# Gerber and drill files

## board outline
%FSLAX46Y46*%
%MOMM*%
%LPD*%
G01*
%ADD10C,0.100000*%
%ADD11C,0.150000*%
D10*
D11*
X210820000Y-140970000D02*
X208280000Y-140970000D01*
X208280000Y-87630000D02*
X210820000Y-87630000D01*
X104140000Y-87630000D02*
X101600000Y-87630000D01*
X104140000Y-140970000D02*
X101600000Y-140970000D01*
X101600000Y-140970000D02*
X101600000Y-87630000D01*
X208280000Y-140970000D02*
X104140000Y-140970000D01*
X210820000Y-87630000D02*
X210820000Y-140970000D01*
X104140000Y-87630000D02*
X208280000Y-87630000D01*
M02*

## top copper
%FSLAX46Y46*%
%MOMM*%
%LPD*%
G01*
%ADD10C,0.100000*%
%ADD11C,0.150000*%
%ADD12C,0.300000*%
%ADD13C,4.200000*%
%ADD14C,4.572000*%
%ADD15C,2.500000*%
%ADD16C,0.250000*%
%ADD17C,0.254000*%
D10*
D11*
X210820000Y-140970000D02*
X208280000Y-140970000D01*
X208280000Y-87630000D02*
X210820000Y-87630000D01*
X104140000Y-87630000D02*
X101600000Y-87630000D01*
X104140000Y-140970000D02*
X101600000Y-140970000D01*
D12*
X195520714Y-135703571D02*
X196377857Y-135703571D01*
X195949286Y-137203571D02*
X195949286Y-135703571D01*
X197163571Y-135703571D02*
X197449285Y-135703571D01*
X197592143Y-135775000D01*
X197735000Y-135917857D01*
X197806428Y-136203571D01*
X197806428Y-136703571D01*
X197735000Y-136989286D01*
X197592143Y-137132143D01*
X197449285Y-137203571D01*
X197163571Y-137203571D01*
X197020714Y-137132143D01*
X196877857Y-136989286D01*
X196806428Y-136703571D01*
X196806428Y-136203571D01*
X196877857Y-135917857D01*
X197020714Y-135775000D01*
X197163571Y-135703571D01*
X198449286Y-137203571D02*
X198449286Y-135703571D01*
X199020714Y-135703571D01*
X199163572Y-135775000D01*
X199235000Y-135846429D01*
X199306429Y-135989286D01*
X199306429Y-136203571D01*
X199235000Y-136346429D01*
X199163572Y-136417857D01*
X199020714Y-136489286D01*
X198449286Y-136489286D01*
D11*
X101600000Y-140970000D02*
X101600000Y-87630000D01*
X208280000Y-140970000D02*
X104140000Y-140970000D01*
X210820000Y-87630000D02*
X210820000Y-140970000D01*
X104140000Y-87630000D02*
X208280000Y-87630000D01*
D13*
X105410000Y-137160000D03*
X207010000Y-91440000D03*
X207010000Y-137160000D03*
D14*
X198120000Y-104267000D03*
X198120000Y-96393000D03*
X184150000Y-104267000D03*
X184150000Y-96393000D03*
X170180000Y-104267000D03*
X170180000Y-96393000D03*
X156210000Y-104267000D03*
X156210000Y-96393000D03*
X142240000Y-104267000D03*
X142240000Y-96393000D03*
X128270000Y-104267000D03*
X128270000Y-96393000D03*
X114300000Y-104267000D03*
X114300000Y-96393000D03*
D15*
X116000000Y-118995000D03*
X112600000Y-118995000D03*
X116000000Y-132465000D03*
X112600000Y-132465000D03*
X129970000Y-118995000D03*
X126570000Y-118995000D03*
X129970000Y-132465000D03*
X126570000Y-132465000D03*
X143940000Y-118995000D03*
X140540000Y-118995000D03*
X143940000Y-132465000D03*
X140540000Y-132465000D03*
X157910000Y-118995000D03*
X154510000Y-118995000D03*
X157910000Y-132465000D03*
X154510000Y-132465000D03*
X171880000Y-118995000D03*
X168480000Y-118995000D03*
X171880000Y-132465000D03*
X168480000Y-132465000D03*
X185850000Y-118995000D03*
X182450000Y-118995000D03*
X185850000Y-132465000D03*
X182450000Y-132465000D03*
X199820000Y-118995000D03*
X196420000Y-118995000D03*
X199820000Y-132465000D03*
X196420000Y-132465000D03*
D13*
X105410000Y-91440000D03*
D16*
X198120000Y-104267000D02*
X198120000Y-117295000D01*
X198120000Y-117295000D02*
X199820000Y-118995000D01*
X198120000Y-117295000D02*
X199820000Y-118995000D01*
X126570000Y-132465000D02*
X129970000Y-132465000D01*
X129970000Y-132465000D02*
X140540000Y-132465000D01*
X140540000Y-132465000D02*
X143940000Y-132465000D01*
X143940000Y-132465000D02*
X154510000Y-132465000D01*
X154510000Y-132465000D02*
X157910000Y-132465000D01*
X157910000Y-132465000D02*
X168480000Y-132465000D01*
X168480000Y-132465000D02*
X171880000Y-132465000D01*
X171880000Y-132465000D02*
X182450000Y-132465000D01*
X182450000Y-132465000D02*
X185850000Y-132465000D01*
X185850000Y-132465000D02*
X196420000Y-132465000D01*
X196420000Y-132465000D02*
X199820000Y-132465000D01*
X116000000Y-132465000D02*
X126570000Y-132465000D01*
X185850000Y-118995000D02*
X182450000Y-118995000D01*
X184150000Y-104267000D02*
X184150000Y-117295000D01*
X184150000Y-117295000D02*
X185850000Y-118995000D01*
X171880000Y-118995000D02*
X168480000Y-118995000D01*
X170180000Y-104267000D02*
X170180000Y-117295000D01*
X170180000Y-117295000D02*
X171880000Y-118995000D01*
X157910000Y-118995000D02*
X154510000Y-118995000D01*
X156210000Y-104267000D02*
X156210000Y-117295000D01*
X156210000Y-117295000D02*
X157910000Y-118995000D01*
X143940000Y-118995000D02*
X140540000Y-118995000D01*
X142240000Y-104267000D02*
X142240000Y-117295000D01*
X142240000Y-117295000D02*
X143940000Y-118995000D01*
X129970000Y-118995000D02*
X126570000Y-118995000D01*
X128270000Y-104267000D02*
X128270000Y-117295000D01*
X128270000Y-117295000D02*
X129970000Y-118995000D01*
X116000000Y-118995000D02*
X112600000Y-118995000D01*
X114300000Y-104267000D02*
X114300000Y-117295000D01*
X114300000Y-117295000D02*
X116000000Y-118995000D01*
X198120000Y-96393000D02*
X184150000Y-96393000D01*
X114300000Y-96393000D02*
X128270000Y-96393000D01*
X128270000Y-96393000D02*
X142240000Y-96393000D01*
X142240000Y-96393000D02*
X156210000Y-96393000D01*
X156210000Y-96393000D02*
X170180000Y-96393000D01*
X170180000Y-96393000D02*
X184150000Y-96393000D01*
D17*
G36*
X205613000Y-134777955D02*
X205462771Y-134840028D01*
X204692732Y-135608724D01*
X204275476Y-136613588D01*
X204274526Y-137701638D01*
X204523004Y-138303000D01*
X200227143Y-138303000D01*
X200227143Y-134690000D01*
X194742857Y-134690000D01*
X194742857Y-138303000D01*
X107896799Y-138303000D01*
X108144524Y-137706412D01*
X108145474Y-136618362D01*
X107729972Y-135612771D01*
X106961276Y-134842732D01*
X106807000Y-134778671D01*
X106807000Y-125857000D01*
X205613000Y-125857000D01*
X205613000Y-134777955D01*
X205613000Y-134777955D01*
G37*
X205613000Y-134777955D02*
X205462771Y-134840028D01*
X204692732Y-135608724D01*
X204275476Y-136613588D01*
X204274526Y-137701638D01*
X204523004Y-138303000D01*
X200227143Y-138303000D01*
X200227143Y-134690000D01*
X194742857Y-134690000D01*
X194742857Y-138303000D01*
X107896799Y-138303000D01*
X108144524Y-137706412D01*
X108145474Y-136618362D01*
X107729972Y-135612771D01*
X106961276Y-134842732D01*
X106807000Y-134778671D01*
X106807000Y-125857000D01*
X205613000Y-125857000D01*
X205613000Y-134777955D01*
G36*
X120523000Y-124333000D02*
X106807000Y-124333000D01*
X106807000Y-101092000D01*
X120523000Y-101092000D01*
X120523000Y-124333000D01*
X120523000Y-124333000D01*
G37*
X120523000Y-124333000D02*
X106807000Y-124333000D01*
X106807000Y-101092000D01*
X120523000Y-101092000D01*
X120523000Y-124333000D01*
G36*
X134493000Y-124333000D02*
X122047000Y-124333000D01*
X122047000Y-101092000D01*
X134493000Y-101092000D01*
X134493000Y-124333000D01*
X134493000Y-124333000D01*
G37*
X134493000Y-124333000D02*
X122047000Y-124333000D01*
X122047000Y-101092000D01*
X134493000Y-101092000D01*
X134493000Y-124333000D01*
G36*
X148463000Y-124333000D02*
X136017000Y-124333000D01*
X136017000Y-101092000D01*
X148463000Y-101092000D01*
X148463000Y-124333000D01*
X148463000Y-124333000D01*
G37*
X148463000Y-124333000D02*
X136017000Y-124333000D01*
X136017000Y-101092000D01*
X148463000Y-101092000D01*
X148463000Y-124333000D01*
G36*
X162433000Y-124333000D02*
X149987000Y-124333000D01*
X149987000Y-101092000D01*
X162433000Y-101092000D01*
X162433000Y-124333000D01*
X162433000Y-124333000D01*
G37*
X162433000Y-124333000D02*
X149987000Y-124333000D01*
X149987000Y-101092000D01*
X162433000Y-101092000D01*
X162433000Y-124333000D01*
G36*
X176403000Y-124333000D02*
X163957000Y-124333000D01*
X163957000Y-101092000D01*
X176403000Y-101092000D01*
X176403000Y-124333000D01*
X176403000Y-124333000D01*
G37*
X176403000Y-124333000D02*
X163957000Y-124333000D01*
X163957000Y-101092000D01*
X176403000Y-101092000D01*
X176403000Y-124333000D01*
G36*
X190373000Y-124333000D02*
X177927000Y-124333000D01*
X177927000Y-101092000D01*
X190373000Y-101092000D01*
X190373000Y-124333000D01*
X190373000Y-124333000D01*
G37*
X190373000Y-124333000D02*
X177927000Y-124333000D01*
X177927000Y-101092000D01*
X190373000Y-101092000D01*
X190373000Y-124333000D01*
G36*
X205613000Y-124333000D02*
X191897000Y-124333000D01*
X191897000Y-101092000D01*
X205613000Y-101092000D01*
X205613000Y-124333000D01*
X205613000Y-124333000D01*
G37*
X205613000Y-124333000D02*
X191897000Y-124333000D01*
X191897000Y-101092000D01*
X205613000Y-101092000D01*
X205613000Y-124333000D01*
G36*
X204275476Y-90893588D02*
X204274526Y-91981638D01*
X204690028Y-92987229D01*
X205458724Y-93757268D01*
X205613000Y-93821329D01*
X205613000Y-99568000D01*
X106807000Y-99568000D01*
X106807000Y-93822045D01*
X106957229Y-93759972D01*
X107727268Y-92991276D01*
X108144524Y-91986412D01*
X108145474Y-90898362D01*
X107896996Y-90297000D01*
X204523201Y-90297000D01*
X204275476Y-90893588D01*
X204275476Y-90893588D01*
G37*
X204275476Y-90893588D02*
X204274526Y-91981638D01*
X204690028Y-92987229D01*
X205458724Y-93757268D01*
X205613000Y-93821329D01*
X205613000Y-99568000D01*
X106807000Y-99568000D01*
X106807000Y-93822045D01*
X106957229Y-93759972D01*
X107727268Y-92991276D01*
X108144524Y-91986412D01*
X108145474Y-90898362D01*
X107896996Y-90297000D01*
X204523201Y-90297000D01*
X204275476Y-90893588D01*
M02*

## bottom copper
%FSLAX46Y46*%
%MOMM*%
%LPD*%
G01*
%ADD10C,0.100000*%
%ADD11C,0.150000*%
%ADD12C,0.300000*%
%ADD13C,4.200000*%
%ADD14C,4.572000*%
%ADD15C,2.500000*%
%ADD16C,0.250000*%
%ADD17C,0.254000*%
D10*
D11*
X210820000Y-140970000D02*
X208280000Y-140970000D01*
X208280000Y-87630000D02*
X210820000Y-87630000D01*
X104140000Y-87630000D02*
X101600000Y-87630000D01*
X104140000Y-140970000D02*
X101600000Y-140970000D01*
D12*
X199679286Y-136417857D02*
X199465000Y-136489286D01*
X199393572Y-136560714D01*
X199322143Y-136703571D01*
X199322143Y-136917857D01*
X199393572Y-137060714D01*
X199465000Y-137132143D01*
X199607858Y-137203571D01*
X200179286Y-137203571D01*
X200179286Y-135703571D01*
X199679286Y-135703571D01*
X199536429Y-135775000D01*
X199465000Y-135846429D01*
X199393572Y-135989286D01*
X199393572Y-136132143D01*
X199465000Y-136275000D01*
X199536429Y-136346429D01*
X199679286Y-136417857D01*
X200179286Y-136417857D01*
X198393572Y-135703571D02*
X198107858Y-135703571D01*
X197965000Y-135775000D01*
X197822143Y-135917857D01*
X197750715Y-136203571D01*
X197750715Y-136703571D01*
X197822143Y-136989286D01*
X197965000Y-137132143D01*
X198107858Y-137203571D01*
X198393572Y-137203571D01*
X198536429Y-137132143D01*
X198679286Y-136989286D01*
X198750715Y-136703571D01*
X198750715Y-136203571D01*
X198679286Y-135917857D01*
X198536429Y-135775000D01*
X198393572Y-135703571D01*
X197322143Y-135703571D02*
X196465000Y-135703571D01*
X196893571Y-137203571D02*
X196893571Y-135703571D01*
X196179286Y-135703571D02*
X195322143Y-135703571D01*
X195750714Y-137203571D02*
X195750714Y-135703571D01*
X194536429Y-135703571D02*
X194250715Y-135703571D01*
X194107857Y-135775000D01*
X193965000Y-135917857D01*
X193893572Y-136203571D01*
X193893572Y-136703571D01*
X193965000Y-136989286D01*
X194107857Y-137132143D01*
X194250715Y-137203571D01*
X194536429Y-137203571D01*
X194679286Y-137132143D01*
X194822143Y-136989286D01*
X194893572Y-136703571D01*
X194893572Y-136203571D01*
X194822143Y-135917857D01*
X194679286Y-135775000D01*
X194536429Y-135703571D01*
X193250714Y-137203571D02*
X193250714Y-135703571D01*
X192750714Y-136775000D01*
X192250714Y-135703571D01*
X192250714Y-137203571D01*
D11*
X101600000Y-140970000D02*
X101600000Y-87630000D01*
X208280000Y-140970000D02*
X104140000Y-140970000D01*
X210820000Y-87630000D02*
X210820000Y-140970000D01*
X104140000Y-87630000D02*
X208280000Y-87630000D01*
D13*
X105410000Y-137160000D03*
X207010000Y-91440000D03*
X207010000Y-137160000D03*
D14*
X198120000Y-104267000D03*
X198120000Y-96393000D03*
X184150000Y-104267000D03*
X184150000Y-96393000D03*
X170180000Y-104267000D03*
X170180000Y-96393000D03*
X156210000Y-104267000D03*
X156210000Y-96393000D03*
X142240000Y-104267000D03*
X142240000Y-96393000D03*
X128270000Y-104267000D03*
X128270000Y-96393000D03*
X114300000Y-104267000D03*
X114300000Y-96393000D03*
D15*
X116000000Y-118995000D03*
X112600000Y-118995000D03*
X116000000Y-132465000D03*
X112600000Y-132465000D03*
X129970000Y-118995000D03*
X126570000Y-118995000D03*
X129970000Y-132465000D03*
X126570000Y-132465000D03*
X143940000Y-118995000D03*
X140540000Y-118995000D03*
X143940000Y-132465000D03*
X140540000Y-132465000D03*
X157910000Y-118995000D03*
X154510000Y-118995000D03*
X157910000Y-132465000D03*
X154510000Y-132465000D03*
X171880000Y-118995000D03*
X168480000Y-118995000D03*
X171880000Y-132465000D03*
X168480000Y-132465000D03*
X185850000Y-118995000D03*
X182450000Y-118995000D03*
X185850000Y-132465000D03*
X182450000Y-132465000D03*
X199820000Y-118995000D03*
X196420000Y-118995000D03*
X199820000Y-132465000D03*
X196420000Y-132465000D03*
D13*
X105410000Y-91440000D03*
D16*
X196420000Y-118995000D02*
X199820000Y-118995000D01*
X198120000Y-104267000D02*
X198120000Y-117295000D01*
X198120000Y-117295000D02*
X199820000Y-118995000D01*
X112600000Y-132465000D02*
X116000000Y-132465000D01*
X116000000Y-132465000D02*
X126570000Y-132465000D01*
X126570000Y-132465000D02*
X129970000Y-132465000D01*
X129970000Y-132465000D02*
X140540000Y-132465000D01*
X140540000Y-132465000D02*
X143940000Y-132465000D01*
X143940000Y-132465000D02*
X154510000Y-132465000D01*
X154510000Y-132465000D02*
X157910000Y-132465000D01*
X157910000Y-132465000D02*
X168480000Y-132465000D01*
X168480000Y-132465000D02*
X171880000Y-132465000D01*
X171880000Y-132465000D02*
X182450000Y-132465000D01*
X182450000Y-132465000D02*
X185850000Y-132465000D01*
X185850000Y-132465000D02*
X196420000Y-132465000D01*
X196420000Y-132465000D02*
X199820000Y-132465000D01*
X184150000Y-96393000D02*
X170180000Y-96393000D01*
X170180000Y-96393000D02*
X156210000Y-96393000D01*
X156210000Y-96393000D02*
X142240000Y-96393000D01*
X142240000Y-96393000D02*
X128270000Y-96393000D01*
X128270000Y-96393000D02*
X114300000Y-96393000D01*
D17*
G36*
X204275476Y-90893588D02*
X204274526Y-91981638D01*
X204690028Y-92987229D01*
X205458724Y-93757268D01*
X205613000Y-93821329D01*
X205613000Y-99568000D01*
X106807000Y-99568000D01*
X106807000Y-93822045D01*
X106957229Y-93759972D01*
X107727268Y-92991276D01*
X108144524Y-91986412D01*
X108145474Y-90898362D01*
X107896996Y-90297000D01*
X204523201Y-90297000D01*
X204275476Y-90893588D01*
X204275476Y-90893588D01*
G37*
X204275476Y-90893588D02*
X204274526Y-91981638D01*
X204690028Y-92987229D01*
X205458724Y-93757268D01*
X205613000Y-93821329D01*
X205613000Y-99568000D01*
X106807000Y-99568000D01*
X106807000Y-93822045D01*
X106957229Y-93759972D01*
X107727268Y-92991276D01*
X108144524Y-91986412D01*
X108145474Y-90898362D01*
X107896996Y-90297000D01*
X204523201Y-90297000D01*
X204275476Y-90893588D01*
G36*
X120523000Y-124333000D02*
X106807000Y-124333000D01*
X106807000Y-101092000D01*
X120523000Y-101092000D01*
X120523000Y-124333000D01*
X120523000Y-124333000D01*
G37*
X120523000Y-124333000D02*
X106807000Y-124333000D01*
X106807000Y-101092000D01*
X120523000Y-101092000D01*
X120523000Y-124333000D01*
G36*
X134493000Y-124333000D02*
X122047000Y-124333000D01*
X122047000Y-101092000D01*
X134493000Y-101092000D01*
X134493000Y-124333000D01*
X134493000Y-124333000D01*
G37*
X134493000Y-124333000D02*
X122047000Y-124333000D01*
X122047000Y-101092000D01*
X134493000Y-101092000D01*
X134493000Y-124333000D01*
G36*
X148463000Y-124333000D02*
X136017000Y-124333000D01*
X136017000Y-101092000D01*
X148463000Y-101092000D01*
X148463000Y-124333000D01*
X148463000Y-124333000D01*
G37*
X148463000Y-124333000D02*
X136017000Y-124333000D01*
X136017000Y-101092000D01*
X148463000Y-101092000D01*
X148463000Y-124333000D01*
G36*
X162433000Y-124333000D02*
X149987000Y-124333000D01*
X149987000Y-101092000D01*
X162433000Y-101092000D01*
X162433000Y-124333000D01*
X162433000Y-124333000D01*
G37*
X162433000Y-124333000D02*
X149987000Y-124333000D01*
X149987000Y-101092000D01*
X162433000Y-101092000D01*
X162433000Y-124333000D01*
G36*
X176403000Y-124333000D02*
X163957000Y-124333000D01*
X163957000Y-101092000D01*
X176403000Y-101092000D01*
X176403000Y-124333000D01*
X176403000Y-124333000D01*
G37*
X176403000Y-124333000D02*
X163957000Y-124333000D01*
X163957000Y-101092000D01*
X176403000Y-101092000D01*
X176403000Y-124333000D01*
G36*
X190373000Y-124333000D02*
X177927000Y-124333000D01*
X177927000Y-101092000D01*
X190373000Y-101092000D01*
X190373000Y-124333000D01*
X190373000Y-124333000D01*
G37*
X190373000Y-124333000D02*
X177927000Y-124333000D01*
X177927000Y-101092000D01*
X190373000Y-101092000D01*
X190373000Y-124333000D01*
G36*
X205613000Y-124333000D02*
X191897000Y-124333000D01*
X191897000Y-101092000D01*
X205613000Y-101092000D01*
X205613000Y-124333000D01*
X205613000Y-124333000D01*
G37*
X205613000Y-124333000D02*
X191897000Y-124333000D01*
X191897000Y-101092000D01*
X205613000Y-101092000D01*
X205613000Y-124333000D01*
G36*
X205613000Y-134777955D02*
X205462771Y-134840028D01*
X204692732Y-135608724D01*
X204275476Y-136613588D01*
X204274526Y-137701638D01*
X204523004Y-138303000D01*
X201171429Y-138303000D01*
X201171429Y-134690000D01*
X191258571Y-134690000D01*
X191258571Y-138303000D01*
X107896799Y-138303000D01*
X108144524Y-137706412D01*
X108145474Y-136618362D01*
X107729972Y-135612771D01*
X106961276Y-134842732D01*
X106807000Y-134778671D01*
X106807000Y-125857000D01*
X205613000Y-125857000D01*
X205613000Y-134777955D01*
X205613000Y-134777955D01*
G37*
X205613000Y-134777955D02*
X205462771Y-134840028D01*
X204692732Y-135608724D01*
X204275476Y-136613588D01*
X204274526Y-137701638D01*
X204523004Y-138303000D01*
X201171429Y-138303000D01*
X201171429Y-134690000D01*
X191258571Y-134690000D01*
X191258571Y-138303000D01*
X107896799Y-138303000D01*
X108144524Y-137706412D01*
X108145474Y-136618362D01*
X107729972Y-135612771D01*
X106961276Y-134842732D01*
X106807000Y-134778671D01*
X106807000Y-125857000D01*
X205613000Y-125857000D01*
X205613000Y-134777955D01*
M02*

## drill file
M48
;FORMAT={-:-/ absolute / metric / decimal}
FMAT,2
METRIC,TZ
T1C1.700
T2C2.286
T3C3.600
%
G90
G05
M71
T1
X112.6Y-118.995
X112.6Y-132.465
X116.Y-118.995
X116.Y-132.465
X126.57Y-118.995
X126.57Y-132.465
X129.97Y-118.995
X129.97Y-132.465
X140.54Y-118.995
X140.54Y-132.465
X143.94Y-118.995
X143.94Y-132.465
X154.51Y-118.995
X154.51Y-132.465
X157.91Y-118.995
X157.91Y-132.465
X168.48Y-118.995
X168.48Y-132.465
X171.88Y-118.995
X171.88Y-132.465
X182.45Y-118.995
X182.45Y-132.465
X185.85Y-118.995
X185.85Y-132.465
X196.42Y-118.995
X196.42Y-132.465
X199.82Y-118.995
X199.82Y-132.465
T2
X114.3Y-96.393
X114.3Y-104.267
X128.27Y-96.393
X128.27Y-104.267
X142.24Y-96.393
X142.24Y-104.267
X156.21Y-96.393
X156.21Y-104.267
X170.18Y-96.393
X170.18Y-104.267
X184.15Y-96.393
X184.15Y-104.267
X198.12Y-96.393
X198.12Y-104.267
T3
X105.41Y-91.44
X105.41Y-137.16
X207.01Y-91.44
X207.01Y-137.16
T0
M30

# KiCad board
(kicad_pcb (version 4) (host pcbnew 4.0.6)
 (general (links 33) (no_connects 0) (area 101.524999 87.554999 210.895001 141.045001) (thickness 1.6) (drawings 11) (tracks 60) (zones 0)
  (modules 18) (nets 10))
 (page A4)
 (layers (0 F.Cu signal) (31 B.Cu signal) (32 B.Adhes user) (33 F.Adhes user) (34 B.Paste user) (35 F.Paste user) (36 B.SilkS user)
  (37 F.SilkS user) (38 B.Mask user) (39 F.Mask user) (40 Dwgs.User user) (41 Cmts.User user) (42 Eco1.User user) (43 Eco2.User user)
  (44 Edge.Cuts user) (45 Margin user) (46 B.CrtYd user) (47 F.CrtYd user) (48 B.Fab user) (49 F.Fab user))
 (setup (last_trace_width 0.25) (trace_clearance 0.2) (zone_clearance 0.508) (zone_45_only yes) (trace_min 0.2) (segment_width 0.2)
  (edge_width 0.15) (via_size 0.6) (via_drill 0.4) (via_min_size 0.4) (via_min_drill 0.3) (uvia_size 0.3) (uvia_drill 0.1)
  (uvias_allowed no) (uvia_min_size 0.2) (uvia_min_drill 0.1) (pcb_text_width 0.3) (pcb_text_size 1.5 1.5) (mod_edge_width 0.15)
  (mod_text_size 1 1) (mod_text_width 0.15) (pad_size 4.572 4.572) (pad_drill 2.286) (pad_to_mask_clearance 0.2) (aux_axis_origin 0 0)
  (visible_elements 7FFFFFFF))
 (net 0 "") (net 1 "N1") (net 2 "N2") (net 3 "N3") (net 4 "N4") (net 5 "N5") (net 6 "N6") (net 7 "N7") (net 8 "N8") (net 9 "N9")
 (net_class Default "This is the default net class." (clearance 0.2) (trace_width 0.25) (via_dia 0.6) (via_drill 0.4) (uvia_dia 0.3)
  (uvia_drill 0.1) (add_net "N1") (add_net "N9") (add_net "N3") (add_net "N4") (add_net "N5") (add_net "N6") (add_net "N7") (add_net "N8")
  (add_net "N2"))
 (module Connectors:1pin (layer F.Cu) (at 105.41 137.16)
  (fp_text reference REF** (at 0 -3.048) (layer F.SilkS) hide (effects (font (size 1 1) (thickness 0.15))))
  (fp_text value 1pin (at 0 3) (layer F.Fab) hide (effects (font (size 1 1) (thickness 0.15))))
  (pad 1 thru_hole circle (at 0 0) (size 4.2 4.2) (drill 3.6) (layers *.Cu *.Mask)))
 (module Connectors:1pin (layer F.Cu) (at 207.01 91.44)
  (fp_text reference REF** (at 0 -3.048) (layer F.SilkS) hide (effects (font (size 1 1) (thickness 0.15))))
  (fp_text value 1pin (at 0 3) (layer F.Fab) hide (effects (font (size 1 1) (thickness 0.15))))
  (pad 1 thru_hole circle (at 0 0) (size 4.2 4.2) (drill 3.6) (layers *.Cu *.Mask)))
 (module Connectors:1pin (layer F.Cu) (at 207.01 137.16)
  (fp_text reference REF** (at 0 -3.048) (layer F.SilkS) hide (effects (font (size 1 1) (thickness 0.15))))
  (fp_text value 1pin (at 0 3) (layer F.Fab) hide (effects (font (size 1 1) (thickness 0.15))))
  (pad 1 thru_hole circle (at 0 0) (size 4.2 4.2) (drill 3.6) (layers *.Cu *.Mask)))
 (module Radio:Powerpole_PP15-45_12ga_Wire (layer F.Cu) (at 198.12 100.33 90)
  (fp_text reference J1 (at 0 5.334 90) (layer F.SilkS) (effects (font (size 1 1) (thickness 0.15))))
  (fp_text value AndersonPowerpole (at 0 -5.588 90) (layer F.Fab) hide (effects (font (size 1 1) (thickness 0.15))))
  (pad 1 thru_hole circle (at -3.937 0 90) (size 4.572 4.572) (drill 2.286) (layers *.Cu *.Mask) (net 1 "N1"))
  (pad 2 thru_hole circle (at 3.937 0 90) (size 4.572 4.572) (drill 2.286) (layers *.Cu *.Mask) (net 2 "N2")))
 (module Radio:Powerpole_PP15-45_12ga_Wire (layer F.Cu) (at 184.15 100.33 90)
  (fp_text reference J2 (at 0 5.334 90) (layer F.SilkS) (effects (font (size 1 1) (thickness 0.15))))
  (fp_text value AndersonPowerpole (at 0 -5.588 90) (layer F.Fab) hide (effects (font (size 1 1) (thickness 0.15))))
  (pad 1 thru_hole circle (at -3.937 0 90) (size 4.572 4.572) (drill 2.286) (layers *.Cu *.Mask) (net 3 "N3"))
  (pad 2 thru_hole circle (at 3.937 0 90) (size 4.572 4.572) (drill 2.286) (layers *.Cu *.Mask) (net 2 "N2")))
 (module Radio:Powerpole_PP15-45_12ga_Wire (layer F.Cu) (at 170.18 100.33 90)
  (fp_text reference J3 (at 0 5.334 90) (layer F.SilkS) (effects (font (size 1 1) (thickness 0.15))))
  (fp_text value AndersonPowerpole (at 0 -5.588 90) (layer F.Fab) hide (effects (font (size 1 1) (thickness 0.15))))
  (pad 1 thru_hole circle (at -3.937 0 90) (size 4.572 4.572) (drill 2.286) (layers *.Cu *.Mask) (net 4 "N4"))
  (pad 2 thru_hole circle (at 3.937 0 90) (size 4.572 4.572) (drill 2.286) (layers *.Cu *.Mask) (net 2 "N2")))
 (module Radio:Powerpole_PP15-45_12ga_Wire (layer F.Cu) (at 156.21 100.33 90)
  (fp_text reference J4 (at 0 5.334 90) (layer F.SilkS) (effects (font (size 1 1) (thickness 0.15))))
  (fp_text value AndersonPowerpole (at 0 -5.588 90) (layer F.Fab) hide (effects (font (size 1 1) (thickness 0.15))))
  (pad 1 thru_hole circle (at -3.937 0 90) (size 4.572 4.572) (drill 2.286) (layers *.Cu *.Mask) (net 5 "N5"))
  (pad 2 thru_hole circle (at 3.937 0 90) (size 4.572 4.572) (drill 2.286) (layers *.Cu *.Mask) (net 2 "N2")))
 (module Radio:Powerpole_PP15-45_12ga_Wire (layer F.Cu) (at 142.24 100.33 90)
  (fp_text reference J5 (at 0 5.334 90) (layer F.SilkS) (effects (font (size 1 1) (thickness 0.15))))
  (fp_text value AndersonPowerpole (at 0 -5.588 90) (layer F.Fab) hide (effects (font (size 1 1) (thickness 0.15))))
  (pad 1 thru_hole circle (at -3.937 0 90) (size 4.572 4.572) (drill 2.286) (layers *.Cu *.Mask) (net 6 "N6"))
  (pad 2 thru_hole circle (at 3.937 0 90) (size 4.572 4.572) (drill 2.286) (layers *.Cu *.Mask) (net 2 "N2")))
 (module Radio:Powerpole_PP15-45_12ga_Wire (layer F.Cu) (at 128.27 100.33 90)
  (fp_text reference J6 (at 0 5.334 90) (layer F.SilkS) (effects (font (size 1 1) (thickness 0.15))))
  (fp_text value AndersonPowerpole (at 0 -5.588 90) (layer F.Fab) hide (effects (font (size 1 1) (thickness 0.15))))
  (pad 1 thru_hole circle (at -3.937 0 90) (size 4.572 4.572) (drill 2.286) (layers *.Cu *.Mask) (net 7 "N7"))
  (pad 2 thru_hole circle (at 3.937 0 90) (size 4.572 4.572) (drill 2.286) (layers *.Cu *.Mask) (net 2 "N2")))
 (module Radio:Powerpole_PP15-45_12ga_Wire (layer F.Cu) (at 114.3 100.33 90)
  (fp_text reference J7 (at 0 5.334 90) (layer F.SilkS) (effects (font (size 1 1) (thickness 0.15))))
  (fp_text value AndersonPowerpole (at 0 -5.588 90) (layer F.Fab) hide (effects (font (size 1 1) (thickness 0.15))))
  (pad 1 thru_hole circle (at -3.937 0 90) (size 4.572 4.572) (drill 2.286) (layers *.Cu *.Mask) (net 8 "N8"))
  (pad 2 thru_hole circle (at 3.937 0 90) (size 4.572 4.572) (drill 2.286) (layers *.Cu *.Mask) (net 2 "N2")))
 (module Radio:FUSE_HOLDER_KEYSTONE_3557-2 (layer F.Cu) (at 114.3 125.73 270)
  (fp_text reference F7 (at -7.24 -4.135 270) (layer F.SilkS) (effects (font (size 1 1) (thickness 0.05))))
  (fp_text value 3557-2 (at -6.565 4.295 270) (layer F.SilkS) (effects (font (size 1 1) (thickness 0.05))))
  (pad 1 thru_hole circle (at -6.735 -1.7 270) (size 2.5 2.5) (drill 1.7) (layers *.Cu *.Mask F.SilkS) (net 8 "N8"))
  (pad 2 thru_hole circle (at -6.735 1.7 270) (size 2.5 2.5) (drill 1.7) (layers *.Cu *.Mask F.SilkS) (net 8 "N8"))
  (pad 3 thru_hole circle (at 6.735 -1.7 270) (size 2.5 2.5) (drill 1.7) (layers *.Cu *.Mask F.SilkS) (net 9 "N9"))
  (pad 4 thru_hole circle (at 6.735 1.7 270) (size 2.5 2.5) (drill 1.7) (layers *.Cu *.Mask F.SilkS) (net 9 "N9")))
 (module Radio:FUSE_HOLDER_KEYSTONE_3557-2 (layer F.Cu) (at 128.27 125.73 270)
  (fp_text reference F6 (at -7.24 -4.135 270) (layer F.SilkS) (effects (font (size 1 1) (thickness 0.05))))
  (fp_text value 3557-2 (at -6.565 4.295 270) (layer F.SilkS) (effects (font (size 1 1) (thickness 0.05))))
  (pad 1 thru_hole circle (at -6.735 -1.7 270) (size 2.5 2.5) (drill 1.7) (layers *.Cu *.Mask F.SilkS) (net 7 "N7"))
  (pad 2 thru_hole circle (at -6.735 1.7 270) (size 2.5 2.5) (drill 1.7) (layers *.Cu *.Mask F.SilkS) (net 7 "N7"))
  (pad 3 thru_hole circle (at 6.735 -1.7 270) (size 2.5 2.5) (drill 1.7) (layers *.Cu *.Mask F.SilkS) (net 9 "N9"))
  (pad 4 thru_hole circle (at 6.735 1.7 270) (size 2.5 2.5) (drill 1.7) (layers *.Cu *.Mask F.SilkS) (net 9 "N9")))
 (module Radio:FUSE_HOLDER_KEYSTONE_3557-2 (layer F.Cu) (at 142.24 125.73 270)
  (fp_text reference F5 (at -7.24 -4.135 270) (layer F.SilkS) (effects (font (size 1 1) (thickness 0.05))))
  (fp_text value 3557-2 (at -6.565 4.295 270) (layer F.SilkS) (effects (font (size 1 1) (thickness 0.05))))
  (pad 1 thru_hole circle (at -6.735 -1.7 270) (size 2.5 2.5) (drill 1.7) (layers *.Cu *.Mask F.SilkS) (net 6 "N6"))
  (pad 2 thru_hole circle (at -6.735 1.7 270) (size 2.5 2.5) (drill 1.7) (layers *.Cu *.Mask F.SilkS) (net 6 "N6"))
  (pad 3 thru_hole circle (at 6.735 -1.7 270) (size 2.5 2.5) (drill 1.7) (layers *.Cu *.Mask F.SilkS) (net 9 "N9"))
  (pad 4 thru_hole circle (at 6.735 1.7 270) (size 2.5 2.5) (drill 1.7) (layers *.Cu *.Mask F.SilkS) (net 9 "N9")))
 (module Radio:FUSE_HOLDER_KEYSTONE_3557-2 (layer F.Cu) (at 156.21 125.73 270)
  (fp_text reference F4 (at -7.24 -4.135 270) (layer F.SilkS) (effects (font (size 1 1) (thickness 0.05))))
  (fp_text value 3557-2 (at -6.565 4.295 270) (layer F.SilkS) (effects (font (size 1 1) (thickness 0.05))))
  (pad 1 thru_hole circle (at -6.735 -1.7 270) (size 2.5 2.5) (drill 1.7) (layers *.Cu *.Mask F.SilkS) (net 5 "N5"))
  (pad 2 thru_hole circle (at -6.735 1.7 270) (size 2.5 2.5) (drill 1.7) (layers *.Cu *.Mask F.SilkS) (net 5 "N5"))
  (pad 3 thru_hole circle (at 6.735 -1.7 270) (size 2.5 2.5) (drill 1.7) (layers *.Cu *.Mask F.SilkS) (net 9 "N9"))
  (pad 4 thru_hole circle (at 6.735 1.7 270) (size 2.5 2.5) (drill 1.7) (layers *.Cu *.Mask F.SilkS) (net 9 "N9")))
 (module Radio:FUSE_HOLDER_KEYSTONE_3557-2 (layer F.Cu) (at 170.18 125.73 270)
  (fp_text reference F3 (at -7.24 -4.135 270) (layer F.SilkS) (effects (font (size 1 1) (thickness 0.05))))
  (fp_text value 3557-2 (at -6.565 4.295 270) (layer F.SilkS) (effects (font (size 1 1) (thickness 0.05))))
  (pad 1 thru_hole circle (at -6.735 -1.7 270) (size 2.5 2.5) (drill 1.7) (layers *.Cu *.Mask F.SilkS) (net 4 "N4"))
  (pad 2 thru_hole circle (at -6.735 1.7 270) (size 2.5 2.5) (drill 1.7) (layers *.Cu *.Mask F.SilkS) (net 4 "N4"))
  (pad 3 thru_hole circle (at 6.735 -1.7 270) (size 2.5 2.5) (drill 1.7) (layers *.Cu *.Mask F.SilkS) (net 9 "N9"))
  (pad 4 thru_hole circle (at 6.735 1.7 270) (size 2.5 2.5) (drill 1.7) (layers *.Cu *.Mask F.SilkS) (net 9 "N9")))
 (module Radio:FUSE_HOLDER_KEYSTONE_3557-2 (layer F.Cu) (at 184.15 125.73 270)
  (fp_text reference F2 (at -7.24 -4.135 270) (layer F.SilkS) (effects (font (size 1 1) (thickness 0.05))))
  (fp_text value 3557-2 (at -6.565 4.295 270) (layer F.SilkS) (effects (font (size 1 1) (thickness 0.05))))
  (pad 1 thru_hole circle (at -6.735 -1.7 270) (size 2.5 2.5) (drill 1.7) (layers *.Cu *.Mask F.SilkS) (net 3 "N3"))
  (pad 2 thru_hole circle (at -6.735 1.7 270) (size 2.5 2.5) (drill 1.7) (layers *.Cu *.Mask F.SilkS) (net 3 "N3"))
  (pad 3 thru_hole circle (at 6.735 -1.7 270) (size 2.5 2.5) (drill 1.7) (layers *.Cu *.Mask F.SilkS) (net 9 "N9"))
  (pad 4 thru_hole circle (at 6.735 1.7 270) (size 2.5 2.5) (drill 1.7) (layers *.Cu *.Mask F.SilkS) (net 9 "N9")))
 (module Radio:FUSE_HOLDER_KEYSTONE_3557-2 (layer F.Cu) (at 198.12 125.73 270)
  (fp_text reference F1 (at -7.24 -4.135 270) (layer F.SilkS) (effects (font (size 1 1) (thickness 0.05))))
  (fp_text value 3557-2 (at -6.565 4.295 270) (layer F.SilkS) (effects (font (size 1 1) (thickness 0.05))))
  (pad 1 thru_hole circle (at -6.735 -1.7 270) (size 2.5 2.5) (drill 1.7) (layers *.Cu *.Mask F.SilkS) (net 1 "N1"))
  (pad 2 thru_hole circle (at -6.735 1.7 270) (size 2.5 2.5) (drill 1.7) (layers *.Cu *.Mask F.SilkS) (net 1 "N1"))
  (pad 3 thru_hole circle (at 6.735 -1.7 270) (size 2.5 2.5) (drill 1.7) (layers *.Cu *.Mask F.SilkS) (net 9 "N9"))
  (pad 4 thru_hole circle (at 6.735 1.7 270) (size 2.5 2.5) (drill 1.7) (layers *.Cu *.Mask F.SilkS) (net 9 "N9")))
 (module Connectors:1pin (layer F.Cu) (at 105.41 91.44)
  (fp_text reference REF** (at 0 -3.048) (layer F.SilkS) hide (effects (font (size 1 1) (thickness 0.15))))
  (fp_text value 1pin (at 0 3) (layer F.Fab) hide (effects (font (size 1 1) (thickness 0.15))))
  (pad 1 thru_hole circle (at 0 0) (size 4.2 4.2) (drill 3.6) (layers *.Cu *.Mask)))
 (gr_line (start 210.82 140.97) (end 208.28 140.97) (angle 90) (layer Edge.Cuts) (width 0.15))
 (gr_line (start 208.28 87.63) (end 210.82 87.63) (angle 90) (layer Edge.Cuts) (width 0.15))
 (gr_line (start 104.14 87.63) (end 101.6 87.63) (angle 90) (layer Edge.Cuts) (width 0.15))
 (gr_line (start 104.14 140.97) (end 101.6 140.97) (angle 90) (layer Edge.Cuts) (width 0.15))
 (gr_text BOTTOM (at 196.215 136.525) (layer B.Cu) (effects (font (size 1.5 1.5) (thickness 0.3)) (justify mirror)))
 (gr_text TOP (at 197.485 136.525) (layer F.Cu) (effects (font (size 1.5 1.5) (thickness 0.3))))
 (gr_line (start 101.6 140.97) (end 101.6 87.63) (angle 90) (layer Edge.Cuts) (width 0.15))
 (gr_line (start 208.28 140.97) (end 104.14 140.97) (angle 90) (layer Edge.Cuts) (width 0.15))
 (gr_line (start 210.82 87.63) (end 210.82 140.97) (angle 90) (layer Edge.Cuts) (width 0.15))
 (gr_line (start 104.14 87.63) (end 208.28 87.63) (angle 90) (layer Edge.Cuts) (width 0.15))
 (segment (start 196.42 118.995) (end 199.82 118.995) (width 0.25) (layer B.Cu) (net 1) (status C00000))
 (segment (start 198.12 104.267) (end 198.12 117.295) (width 0.25) (layer F.Cu) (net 1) (status 400000))
 (segment (start 198.12 104.267) (end 198.12 117.295) (width 0.25) (layer B.Cu) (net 1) (status 400000))
 (segment (start 198.12 117.295) (end 199.82 118.995) (width 0.25) (layer B.Cu) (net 1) (status 800000))
 (segment (start 198.12 117.295) (end 199.82 118.995) (width 0.25) (layer F.Cu) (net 1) (status 800000))
 (segment (start 198.12 117.295) (end 199.82 118.995) (width 0.25) (layer F.Cu) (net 1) (status 800000))
 (segment (start 112.6 132.465) (end 116 132.465) (width 0.25) (layer B.Cu) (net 9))
 (segment (start 116 132.465) (end 126.57 132.465) (width 0.25) (layer B.Cu) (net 9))
 (segment (start 126.57 132.465) (end 129.97 132.465) (width 0.25) (layer B.Cu) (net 9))
 (segment (start 129.97 132.465) (end 140.54 132.465) (width 0.25) (layer B.Cu) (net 9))
 (segment (start 140.54 132.465) (end 143.94 132.465) (width 0.25) (layer B.Cu) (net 9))
 (segment (start 143.94 132.465) (end 154.51 132.465) (width 0.25) (layer B.Cu) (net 9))
 (segment (start 154.51 132.465) (end 157.91 132.465) (width 0.25) (layer B.Cu) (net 9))
 (segment (start 157.91 132.465) (end 168.48 132.465) (width 0.25) (layer B.Cu) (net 9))
 (segment (start 168.48 132.465) (end 171.88 132.465) (width 0.25) (layer B.Cu) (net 9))
 (segment (start 171.88 132.465) (end 182.45 132.465) (width 0.25) (layer B.Cu) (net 9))
 (segment (start 182.45 132.465) (end 185.85 132.465) (width 0.25) (layer B.Cu) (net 9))
 (segment (start 185.85 132.465) (end 196.42 132.465) (width 0.25) (layer B.Cu) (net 9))
 (segment (start 196.42 132.465) (end 199.82 132.465) (width 0.25) (layer B.Cu) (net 9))
 (segment (start 126.57 132.465) (end 129.97 132.465) (width 0.25) (layer F.Cu) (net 9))
 (segment (start 129.97 132.465) (end 140.54 132.465) (width 0.25) (layer F.Cu) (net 9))
 (segment (start 140.54 132.465) (end 143.94 132.465) (width 0.25) (layer F.Cu) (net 9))
 (segment (start 143.94 132.465) (end 154.51 132.465) (width 0.25) (layer F.Cu) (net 9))
 (segment (start 154.51 132.465) (end 157.91 132.465) (width 0.25) (layer F.Cu) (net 9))
 (segment (start 157.91 132.465) (end 168.48 132.465) (width 0.25) (layer F.Cu) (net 9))
 (segment (start 168.48 132.465) (end 171.88 132.465) (width 0.25) (layer F.Cu) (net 9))
 (segment (start 171.88 132.465) (end 182.45 132.465) (width 0.25) (layer F.Cu) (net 9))
 (segment (start 182.45 132.465) (end 185.85 132.465) (width 0.25) (layer F.Cu) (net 9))
 (segment (start 185.85 132.465) (end 196.42 132.465) (width 0.25) (layer F.Cu) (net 9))
 (segment (start 196.42 132.465) (end 199.82 132.465) (width 0.25) (layer F.Cu) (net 9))
 (segment (start 116 132.465) (end 126.57 132.465) (width 0.25) (layer F.Cu) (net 9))
 (segment (start 185.85 118.995) (end 182.45 118.995) (width 0.25) (layer F.Cu) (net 3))
 (segment (start 184.15 104.267) (end 184.15 117.295) (width 0.25) (layer F.Cu) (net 3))
 (segment (start 184.15 117.295) (end 185.85 118.995) (width 0.25) (layer F.Cu) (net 3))
 (segment (start 171.88 118.995) (end 168.48 118.995) (width 0.25) (layer F.Cu) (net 4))
 (segment (start 170.18 104.267) (end 170.18 117.295) (width 0.25) (layer F.Cu) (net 4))
 (segment (start 170.18 117.295) (end 171.88 118.995) (width 0.25) (layer F.Cu) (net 4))
 (segment (start 157.91 118.995) (end 154.51 118.995) (width 0.25) (layer F.Cu) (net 5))
 (segment (start 156.21 104.267) (end 156.21 117.295) (width 0.25) (layer F.Cu) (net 5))
 (segment (start 156.21 117.295) (end 157.91 118.995) (width 0.25) (layer F.Cu) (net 5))
 (segment (start 143.94 118.995) (end 140.54 118.995) (width 0.25) (layer F.Cu) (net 6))
 (segment (start 142.24 104.267) (end 142.24 117.295) (width 0.25) (layer F.Cu) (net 6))
 (segment (start 142.24 117.295) (end 143.94 118.995) (width 0.25) (layer F.Cu) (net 6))
 (segment (start 129.97 118.995) (end 126.57 118.995) (width 0.25) (layer F.Cu) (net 7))
 (segment (start 128.27 104.267) (end 128.27 117.295) (width 0.25) (layer F.Cu) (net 7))
 (segment (start 128.27 117.295) (end 129.97 118.995) (width 0.25) (layer F.Cu) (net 7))
 (segment (start 116 118.995) (end 112.6 118.995) (width 0.25) (layer F.Cu) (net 8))
 (segment (start 114.3 104.267) (end 114.3 117.295) (width 0.25) (layer F.Cu) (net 8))
 (segment (start 114.3 117.295) (end 116 118.995) (width 0.25) (layer F.Cu) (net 8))
 (segment (start 198.12 96.393) (end 184.15 96.393) (width 0.25) (layer F.Cu) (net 2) (status C00000))
 (segment (start 184.15 96.393) (end 170.18 96.393) (width 0.25) (layer B.Cu) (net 2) (status C00000))
 (segment (start 170.18 96.393) (end 156.21 96.393) (width 0.25) (layer B.Cu) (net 2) (status C00000))
 (segment (start 156.21 96.393) (end 142.24 96.393) (width 0.25) (layer B.Cu) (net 2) (status C00000))
 (segment (start 142.24 96.393) (end 128.27 96.393) (width 0.25) (layer B.Cu) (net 2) (status C00000))
 (segment (start 128.27 96.393) (end 114.3 96.393) (width 0.25) (layer B.Cu) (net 2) (status C00000))
 (segment (start 114.3 96.393) (end 128.27 96.393) (width 0.25) (layer F.Cu) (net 2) (status C00000))
 (segment (start 128.27 96.393) (end 142.24 96.393) (width 0.25) (layer F.Cu) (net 2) (status C00000))
 (segment (start 142.24 96.393) (end 156.21 96.393) (width 0.25) (layer F.Cu) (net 2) (status C00000))
 (segment (start 156.21 96.393) (end 170.18 96.393) (width 0.25) (layer F.Cu) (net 2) (status C00000))
 (segment (start 170.18 96.393) (end 184.15 96.393) (width 0.25) (layer F.Cu) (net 2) (status C00000))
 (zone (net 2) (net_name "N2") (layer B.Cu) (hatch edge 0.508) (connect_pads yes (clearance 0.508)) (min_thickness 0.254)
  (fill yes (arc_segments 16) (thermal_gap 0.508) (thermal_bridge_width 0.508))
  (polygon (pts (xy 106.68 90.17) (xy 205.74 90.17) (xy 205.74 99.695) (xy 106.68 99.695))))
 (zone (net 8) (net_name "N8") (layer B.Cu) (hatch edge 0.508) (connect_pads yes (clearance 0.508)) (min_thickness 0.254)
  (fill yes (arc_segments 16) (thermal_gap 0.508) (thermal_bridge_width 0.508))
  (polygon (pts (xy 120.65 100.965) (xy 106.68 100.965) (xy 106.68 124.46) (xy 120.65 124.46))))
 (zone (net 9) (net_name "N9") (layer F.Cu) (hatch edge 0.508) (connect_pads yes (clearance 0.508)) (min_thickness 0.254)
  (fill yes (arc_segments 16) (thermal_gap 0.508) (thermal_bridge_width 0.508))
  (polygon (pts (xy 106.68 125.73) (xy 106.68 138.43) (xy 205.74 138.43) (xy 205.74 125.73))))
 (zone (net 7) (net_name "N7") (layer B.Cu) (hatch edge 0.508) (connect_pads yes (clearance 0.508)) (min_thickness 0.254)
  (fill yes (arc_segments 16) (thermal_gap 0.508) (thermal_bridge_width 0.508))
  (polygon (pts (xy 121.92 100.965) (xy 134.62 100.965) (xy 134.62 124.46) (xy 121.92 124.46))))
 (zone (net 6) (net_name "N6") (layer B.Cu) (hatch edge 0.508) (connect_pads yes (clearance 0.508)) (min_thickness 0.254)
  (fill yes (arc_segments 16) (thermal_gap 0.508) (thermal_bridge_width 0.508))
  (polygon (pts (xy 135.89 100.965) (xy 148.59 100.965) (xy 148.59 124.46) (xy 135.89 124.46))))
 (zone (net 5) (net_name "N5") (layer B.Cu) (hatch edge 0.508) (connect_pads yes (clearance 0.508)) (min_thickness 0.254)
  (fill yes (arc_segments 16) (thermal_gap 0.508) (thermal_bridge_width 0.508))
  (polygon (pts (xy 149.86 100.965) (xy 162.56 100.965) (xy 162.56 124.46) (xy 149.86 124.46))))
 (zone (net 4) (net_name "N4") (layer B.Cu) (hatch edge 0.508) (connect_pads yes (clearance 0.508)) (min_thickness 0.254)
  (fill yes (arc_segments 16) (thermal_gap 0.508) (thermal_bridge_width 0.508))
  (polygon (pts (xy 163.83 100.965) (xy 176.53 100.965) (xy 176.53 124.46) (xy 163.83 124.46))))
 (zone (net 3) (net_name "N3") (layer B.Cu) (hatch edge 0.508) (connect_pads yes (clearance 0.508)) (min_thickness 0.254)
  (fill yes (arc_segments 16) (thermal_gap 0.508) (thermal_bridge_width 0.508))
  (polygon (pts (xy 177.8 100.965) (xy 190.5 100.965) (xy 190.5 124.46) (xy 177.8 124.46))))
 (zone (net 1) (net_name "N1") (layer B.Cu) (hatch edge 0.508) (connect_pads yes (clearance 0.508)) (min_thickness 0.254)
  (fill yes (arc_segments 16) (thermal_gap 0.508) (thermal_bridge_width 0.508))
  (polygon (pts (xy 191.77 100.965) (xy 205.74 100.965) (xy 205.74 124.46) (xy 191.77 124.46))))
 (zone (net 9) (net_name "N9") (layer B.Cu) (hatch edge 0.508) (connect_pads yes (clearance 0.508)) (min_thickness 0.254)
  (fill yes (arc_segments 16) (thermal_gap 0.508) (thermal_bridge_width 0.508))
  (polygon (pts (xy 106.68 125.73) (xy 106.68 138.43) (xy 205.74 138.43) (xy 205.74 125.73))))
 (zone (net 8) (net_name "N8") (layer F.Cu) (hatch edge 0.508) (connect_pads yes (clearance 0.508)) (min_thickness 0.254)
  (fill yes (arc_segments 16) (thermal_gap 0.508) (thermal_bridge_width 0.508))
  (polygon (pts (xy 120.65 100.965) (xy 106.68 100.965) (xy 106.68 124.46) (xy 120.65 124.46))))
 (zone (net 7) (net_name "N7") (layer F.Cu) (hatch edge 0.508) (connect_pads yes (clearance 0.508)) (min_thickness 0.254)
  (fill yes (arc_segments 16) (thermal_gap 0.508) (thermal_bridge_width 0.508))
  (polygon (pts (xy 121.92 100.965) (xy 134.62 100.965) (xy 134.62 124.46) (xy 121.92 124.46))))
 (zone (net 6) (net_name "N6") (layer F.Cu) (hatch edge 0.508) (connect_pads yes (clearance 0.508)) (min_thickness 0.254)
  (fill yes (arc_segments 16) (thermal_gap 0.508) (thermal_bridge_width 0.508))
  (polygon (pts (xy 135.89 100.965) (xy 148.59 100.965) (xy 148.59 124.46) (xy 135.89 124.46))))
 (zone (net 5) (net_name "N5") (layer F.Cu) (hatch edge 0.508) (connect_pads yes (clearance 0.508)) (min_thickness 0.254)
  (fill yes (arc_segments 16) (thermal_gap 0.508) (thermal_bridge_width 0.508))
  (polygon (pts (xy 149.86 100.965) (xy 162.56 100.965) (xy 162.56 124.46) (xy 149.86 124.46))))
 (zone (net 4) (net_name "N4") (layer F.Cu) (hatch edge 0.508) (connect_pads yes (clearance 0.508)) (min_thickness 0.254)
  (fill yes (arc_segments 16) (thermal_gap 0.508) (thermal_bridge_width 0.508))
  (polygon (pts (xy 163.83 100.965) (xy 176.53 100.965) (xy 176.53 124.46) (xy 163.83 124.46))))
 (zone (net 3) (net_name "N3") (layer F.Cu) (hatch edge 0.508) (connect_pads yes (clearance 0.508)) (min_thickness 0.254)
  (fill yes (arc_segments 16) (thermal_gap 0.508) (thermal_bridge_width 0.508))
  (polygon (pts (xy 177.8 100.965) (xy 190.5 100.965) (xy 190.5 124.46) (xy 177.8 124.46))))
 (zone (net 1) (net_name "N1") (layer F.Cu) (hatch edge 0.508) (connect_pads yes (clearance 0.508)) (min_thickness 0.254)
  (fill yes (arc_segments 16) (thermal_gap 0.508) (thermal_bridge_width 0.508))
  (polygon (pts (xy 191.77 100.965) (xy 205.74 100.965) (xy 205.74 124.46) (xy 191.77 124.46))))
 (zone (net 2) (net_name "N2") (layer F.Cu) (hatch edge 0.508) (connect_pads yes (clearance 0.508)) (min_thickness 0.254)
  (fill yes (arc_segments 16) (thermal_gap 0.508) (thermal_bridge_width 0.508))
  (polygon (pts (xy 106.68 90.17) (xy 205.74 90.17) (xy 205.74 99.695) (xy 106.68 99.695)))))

